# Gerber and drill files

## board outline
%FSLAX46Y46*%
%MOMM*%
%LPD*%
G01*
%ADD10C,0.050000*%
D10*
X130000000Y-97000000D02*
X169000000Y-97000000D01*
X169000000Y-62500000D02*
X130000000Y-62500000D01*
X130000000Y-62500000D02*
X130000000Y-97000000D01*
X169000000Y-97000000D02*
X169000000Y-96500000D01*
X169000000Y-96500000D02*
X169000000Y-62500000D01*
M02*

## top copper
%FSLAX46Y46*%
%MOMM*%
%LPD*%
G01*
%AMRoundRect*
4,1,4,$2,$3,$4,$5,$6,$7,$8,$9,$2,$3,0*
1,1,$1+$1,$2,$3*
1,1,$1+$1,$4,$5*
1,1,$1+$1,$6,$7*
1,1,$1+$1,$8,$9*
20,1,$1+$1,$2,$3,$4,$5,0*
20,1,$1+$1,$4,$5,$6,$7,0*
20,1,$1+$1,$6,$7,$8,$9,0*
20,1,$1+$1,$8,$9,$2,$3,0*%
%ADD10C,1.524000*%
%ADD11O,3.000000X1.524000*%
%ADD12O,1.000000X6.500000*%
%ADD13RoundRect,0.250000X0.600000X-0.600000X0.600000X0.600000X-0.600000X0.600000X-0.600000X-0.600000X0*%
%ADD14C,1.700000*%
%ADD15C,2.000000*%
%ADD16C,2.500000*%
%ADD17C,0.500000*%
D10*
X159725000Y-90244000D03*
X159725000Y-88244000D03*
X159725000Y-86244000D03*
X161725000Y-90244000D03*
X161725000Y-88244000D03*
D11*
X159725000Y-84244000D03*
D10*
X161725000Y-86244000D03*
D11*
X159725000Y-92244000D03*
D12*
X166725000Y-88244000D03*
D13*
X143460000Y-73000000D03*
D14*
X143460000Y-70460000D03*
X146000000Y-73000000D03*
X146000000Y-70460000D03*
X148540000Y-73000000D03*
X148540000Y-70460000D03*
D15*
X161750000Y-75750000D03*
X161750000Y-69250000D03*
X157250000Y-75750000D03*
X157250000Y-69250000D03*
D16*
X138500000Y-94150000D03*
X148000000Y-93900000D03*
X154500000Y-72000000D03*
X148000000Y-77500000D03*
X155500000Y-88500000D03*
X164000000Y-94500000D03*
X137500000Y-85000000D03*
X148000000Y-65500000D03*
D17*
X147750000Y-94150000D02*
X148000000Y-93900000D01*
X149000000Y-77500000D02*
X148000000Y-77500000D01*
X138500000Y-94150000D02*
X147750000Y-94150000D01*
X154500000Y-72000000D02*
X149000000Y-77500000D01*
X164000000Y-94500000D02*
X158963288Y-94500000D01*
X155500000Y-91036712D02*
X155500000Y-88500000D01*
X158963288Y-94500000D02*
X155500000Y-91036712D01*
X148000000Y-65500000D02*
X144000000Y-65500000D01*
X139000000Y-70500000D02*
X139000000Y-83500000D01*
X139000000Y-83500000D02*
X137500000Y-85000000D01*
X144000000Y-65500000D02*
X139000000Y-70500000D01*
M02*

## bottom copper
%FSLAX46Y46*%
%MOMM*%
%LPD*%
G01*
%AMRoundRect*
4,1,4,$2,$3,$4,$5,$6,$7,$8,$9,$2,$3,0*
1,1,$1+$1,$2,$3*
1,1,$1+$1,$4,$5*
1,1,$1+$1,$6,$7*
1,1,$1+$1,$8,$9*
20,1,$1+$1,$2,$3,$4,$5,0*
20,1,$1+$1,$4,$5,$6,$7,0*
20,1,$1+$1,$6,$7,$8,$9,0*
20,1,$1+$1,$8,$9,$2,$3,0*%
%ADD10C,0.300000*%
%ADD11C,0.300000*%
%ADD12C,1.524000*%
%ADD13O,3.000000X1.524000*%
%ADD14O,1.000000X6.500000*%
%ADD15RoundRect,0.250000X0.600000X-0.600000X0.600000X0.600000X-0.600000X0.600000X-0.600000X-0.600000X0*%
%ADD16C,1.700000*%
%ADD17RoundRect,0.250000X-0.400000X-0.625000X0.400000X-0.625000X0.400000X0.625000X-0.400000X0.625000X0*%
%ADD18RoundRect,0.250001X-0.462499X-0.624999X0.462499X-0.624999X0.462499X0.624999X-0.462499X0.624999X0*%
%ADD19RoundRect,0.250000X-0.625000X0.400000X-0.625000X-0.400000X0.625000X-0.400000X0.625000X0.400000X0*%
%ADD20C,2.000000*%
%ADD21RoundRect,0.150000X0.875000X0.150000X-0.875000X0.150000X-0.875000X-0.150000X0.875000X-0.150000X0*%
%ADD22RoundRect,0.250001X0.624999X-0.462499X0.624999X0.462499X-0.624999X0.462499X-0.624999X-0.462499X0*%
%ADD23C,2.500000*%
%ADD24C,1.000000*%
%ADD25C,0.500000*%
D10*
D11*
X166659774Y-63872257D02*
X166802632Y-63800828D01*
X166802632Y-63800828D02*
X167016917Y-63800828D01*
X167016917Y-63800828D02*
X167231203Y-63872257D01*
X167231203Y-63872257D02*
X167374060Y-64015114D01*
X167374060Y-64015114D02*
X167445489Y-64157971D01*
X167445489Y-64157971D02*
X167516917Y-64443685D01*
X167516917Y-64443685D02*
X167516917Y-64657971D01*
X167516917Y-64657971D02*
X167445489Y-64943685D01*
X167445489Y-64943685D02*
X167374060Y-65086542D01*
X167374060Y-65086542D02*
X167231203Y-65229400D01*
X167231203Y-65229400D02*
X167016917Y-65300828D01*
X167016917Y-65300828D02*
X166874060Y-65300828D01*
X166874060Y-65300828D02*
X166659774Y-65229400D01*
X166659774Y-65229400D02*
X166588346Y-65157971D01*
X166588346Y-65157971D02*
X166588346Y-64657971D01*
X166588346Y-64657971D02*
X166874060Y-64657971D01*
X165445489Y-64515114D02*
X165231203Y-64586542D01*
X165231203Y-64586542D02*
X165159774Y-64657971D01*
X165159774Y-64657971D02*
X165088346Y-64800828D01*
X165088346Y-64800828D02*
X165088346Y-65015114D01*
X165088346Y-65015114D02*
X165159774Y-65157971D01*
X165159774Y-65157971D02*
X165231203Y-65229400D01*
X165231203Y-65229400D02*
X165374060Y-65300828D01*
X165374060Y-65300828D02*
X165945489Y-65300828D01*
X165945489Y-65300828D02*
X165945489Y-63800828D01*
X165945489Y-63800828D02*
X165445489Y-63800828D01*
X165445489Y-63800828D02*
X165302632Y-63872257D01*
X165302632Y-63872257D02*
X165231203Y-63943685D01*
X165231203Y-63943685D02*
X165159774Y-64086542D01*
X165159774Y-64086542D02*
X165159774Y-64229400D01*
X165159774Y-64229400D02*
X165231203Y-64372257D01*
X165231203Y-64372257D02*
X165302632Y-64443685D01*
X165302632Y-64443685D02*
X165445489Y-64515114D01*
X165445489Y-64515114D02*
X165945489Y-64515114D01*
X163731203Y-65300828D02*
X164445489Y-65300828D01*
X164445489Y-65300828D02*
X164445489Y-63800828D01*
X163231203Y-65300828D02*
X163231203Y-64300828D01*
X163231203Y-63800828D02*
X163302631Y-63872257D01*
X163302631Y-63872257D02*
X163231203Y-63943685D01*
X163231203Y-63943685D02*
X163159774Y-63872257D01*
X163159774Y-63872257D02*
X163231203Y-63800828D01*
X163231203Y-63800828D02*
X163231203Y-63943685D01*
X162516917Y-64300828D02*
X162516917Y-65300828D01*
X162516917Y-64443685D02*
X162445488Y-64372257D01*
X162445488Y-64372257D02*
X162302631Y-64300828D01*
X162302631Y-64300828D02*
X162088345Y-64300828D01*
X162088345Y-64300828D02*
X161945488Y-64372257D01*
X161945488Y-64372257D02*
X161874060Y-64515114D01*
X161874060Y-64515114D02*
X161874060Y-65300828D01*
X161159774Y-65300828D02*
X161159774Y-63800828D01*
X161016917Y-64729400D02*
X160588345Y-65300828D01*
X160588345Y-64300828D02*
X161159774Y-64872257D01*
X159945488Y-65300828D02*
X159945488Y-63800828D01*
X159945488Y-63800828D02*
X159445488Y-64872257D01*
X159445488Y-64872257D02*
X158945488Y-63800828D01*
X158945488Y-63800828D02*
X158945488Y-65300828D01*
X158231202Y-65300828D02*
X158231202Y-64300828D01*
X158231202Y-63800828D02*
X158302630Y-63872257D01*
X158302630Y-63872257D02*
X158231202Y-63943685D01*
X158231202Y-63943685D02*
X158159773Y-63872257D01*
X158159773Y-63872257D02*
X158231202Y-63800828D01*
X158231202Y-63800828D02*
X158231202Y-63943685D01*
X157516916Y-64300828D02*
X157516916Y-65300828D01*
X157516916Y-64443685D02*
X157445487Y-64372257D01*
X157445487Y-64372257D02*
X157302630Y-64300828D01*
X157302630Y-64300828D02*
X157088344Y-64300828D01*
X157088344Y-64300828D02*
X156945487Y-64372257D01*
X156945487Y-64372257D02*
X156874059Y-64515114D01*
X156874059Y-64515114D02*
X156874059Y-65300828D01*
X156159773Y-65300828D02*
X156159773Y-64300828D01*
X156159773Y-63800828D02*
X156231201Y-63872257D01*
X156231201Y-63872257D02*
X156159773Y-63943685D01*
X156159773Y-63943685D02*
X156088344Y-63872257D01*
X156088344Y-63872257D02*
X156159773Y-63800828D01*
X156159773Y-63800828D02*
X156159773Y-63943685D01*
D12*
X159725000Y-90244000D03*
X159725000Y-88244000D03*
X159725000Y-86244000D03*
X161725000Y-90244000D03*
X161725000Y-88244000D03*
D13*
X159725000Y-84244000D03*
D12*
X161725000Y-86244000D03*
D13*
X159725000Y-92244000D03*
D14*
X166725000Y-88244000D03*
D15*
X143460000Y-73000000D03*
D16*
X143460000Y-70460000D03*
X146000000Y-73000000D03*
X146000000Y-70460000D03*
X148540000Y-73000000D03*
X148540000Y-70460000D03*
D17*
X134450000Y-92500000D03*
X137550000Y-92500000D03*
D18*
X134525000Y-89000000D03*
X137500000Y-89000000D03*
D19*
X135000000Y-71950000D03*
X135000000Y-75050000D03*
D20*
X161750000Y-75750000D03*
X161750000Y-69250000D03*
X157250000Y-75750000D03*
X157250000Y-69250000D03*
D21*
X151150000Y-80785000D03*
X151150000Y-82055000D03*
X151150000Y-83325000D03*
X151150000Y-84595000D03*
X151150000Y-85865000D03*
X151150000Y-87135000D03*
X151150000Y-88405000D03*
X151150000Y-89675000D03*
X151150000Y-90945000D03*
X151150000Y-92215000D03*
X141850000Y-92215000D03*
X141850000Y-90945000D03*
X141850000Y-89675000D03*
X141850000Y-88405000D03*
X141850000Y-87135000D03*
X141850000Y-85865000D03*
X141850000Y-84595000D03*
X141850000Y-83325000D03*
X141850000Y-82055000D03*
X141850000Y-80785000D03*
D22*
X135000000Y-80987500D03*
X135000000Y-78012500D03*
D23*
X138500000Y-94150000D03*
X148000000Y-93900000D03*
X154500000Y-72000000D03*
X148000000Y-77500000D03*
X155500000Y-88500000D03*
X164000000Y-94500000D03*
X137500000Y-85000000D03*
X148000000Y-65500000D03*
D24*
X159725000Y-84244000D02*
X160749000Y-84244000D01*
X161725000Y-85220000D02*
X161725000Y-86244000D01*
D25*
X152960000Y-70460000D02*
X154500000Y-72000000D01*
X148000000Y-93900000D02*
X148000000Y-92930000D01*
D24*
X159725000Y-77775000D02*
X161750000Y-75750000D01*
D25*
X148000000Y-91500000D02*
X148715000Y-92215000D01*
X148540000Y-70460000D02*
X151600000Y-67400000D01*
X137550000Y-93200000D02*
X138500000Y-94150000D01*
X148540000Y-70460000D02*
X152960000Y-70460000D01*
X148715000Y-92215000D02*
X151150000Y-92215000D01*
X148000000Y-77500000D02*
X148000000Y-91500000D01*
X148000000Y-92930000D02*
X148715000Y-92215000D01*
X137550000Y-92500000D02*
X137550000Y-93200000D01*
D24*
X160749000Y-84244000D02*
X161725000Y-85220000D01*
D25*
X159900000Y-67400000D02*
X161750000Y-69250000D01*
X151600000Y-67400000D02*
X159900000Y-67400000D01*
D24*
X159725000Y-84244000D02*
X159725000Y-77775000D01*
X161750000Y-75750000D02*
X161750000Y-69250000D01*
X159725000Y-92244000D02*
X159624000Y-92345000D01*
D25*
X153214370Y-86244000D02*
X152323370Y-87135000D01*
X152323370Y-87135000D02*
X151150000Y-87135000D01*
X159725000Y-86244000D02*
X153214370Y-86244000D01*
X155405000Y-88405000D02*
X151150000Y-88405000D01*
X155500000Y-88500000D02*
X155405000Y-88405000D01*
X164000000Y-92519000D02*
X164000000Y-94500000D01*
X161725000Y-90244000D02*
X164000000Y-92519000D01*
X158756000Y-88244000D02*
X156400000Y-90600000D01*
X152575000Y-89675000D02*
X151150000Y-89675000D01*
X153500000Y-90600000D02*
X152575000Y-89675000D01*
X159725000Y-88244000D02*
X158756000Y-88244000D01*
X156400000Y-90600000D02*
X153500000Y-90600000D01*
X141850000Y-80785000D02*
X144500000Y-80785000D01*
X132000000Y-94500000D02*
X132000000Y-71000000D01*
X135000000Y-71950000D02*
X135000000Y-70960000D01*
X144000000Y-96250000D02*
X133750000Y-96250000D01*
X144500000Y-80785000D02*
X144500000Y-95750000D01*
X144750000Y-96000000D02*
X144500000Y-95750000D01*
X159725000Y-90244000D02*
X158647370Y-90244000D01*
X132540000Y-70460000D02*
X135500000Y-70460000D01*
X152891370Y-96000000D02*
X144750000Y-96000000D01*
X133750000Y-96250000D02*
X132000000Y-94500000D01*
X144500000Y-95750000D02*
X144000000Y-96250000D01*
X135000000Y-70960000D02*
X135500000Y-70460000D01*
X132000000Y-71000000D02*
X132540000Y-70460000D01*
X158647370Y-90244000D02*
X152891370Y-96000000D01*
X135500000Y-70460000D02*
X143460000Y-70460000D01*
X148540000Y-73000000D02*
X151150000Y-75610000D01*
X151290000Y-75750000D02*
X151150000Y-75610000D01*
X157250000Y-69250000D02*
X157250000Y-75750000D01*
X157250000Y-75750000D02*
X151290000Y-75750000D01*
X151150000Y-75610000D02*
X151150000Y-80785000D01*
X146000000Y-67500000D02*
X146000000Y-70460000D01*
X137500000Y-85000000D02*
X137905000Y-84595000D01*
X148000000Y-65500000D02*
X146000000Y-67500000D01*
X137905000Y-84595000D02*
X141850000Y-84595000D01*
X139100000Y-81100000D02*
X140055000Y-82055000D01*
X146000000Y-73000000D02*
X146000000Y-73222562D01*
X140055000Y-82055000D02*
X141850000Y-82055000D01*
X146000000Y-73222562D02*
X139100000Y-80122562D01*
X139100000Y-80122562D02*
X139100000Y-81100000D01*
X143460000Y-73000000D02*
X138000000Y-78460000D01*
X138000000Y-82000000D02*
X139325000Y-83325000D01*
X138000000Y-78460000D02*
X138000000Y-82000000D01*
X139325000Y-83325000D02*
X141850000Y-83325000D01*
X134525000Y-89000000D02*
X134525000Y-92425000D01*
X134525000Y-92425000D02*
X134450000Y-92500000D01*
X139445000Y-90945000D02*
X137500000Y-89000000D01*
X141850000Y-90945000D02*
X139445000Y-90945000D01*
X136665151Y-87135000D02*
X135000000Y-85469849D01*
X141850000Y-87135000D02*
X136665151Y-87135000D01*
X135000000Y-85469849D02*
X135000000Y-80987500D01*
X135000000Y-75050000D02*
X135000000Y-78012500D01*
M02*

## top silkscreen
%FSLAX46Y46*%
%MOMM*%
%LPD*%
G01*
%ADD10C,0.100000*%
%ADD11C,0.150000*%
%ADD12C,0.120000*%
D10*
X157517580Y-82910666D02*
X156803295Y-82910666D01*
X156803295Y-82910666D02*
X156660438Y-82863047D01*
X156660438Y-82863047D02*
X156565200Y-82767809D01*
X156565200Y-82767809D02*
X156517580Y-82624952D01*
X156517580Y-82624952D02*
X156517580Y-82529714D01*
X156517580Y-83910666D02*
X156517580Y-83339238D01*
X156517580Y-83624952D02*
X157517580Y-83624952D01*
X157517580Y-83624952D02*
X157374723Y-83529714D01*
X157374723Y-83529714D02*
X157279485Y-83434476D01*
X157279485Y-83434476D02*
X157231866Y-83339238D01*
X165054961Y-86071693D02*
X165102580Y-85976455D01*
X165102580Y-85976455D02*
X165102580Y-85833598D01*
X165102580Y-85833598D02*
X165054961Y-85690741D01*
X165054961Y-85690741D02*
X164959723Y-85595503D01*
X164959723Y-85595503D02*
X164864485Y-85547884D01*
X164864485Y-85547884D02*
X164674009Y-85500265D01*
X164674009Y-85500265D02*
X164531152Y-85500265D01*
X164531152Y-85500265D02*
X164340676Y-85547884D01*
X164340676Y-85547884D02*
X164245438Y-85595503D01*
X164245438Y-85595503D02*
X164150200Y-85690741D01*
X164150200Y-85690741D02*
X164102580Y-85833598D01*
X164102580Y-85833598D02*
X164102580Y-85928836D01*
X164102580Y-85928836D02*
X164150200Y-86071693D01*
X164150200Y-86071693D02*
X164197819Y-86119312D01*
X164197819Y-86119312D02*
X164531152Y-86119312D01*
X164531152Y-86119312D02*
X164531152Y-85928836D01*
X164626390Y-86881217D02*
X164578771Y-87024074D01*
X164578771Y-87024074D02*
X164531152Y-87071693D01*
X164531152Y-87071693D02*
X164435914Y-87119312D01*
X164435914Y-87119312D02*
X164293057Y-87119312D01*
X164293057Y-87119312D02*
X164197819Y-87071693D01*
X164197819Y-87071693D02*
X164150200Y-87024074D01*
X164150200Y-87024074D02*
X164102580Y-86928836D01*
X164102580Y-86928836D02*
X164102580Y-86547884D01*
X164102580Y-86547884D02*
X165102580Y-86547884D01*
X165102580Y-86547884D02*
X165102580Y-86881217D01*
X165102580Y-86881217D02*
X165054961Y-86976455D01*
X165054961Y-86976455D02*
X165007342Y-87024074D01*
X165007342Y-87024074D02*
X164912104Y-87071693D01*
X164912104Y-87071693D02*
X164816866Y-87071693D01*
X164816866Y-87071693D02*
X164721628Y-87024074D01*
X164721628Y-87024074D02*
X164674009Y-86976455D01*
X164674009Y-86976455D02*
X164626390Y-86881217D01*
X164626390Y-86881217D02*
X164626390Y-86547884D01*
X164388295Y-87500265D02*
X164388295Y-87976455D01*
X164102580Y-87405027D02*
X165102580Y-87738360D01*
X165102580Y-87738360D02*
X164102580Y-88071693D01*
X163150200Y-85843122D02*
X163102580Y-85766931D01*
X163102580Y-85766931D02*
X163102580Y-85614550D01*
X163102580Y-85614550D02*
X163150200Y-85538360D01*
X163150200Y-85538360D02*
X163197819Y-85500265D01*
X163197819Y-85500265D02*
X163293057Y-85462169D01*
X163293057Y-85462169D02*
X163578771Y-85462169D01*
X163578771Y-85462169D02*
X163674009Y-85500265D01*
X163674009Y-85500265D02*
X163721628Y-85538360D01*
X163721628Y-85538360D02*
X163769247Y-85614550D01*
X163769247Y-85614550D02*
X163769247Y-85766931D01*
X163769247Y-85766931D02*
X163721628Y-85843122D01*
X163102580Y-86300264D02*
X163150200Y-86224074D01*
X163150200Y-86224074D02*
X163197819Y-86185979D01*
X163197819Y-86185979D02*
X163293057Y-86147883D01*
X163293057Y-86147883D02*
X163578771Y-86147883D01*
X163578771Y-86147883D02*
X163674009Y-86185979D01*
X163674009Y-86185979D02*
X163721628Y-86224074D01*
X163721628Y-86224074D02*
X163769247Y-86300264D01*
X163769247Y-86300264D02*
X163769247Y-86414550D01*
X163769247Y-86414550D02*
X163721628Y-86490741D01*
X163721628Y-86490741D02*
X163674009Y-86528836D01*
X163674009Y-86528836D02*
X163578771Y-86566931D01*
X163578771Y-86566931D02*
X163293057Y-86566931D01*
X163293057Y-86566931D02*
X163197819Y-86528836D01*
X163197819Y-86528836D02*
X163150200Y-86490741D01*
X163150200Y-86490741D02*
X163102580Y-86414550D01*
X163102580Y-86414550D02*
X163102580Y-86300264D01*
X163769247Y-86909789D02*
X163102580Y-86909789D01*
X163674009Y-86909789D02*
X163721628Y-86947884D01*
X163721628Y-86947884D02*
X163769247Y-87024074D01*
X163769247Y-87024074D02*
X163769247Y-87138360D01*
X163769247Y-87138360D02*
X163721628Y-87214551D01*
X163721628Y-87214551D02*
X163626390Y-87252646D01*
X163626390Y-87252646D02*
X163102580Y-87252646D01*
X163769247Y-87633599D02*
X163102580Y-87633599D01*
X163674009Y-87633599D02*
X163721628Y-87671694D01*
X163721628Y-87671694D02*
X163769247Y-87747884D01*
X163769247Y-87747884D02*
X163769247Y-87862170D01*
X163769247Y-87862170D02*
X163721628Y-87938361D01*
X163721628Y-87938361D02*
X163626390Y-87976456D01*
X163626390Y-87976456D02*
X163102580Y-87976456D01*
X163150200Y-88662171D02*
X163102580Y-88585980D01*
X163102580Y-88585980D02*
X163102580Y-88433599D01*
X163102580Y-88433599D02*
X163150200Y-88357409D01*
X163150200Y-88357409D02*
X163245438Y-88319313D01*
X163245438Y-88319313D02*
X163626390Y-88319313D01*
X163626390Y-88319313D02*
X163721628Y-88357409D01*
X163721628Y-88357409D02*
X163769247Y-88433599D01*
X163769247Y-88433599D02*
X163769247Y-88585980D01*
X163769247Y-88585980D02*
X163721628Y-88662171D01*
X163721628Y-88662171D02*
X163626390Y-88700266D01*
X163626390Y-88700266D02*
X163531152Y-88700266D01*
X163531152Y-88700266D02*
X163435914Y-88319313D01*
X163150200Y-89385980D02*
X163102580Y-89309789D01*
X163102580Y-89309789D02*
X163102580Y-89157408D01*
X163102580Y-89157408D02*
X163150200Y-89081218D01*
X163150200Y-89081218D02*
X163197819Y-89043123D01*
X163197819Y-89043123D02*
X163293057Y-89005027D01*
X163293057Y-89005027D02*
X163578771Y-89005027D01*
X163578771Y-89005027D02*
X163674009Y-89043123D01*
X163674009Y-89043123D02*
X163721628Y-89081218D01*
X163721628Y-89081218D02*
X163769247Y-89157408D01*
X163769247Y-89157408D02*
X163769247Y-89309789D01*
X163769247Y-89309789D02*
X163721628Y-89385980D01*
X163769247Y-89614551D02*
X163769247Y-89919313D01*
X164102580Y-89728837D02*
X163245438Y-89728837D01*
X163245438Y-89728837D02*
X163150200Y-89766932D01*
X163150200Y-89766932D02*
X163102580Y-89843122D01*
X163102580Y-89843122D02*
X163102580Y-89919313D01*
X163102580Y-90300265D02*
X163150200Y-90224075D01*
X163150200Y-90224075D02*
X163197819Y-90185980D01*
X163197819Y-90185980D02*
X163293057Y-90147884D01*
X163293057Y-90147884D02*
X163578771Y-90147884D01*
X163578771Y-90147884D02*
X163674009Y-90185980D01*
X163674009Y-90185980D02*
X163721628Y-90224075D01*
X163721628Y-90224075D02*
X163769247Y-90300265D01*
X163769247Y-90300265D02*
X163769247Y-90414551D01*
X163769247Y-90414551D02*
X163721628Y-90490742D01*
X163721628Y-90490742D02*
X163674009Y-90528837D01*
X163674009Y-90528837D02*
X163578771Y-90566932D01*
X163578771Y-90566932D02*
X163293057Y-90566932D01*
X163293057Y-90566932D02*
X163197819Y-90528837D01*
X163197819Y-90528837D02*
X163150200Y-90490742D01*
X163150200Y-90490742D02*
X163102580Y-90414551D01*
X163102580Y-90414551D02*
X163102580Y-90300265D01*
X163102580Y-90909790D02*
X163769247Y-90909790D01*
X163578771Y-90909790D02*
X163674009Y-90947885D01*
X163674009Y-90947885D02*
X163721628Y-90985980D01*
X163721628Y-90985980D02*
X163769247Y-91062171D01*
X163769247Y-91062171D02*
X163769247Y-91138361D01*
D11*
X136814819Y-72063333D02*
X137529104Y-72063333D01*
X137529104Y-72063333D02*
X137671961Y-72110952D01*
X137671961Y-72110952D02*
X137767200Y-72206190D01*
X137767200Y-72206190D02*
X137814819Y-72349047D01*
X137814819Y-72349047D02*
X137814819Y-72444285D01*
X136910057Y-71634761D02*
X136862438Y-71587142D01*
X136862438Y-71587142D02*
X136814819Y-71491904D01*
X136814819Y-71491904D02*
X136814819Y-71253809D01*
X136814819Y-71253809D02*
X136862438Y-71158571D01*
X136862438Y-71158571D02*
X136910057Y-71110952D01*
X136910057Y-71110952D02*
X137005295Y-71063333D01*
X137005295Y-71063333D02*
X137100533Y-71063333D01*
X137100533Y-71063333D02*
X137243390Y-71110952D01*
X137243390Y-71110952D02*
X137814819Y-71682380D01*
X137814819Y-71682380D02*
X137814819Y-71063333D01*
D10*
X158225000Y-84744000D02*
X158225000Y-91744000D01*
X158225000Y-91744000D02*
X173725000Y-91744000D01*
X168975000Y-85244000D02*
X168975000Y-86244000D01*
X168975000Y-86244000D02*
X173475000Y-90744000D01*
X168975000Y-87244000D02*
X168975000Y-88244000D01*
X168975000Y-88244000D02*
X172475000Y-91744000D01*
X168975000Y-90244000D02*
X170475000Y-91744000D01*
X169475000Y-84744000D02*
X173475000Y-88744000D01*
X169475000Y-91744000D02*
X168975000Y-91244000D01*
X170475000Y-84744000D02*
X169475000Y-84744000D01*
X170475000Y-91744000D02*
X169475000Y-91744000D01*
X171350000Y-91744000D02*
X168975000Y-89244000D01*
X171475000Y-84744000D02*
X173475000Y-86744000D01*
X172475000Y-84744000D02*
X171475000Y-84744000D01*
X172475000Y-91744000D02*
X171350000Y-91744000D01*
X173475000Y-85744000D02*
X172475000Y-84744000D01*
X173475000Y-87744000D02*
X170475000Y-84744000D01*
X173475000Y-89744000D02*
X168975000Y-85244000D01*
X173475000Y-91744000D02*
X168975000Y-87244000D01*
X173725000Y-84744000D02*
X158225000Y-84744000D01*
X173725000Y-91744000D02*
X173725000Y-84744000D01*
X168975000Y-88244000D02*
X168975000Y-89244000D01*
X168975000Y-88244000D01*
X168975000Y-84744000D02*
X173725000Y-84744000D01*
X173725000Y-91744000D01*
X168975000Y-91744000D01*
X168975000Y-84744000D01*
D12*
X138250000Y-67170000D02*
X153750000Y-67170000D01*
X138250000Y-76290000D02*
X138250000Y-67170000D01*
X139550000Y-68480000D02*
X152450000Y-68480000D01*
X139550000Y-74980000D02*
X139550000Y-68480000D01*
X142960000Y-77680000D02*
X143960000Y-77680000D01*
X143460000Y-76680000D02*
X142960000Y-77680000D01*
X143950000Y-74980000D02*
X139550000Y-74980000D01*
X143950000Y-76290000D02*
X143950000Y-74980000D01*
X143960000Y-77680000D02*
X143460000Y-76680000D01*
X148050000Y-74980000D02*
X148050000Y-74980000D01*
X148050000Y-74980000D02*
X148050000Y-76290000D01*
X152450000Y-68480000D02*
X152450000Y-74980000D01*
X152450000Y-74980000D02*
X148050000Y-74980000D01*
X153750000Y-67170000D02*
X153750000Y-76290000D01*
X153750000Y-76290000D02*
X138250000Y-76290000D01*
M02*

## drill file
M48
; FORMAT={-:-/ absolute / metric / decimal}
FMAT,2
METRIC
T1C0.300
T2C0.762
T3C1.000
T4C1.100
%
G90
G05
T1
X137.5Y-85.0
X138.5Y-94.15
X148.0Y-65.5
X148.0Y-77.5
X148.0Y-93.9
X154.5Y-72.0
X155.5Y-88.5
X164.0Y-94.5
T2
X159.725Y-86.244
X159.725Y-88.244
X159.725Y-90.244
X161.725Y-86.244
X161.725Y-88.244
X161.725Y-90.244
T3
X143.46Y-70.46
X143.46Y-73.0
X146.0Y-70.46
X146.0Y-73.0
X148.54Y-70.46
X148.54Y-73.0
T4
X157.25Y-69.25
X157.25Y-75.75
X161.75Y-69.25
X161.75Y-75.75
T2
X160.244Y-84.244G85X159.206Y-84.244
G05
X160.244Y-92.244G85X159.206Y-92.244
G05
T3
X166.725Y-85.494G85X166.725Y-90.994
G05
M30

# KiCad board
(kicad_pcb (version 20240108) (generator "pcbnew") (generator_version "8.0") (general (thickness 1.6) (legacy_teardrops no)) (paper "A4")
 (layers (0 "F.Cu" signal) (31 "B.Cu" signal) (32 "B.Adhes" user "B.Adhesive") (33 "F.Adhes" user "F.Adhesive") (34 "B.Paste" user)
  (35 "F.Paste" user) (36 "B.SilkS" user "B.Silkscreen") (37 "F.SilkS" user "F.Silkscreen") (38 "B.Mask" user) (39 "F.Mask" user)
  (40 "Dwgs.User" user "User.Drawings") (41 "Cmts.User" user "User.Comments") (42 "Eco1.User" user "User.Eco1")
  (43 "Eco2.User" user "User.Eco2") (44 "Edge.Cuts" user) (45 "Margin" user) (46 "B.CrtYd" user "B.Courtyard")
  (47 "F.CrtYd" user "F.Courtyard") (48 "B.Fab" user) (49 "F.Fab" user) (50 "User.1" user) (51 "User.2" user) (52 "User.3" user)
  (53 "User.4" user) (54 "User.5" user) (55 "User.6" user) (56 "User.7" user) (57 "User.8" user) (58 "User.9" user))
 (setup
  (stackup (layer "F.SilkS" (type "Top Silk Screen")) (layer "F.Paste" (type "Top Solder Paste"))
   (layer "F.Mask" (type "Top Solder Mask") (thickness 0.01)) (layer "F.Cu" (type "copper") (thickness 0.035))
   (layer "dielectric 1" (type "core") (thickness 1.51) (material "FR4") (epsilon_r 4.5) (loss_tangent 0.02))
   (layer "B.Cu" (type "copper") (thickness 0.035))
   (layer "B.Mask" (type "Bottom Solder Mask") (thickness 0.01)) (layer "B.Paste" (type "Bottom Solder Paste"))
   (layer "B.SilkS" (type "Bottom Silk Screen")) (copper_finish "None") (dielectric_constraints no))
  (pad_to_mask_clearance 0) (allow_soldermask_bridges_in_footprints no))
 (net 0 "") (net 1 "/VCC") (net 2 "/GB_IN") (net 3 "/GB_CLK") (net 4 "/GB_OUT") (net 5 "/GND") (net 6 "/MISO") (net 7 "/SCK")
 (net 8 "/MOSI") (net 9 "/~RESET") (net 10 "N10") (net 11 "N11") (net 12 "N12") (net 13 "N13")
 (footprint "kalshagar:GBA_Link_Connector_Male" (layer "F.Cu") (at 156.475 83.244 -90)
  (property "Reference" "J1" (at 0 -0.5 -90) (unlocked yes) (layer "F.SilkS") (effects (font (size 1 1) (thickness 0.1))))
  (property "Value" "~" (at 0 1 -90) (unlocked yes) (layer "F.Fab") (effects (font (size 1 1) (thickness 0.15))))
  (fp_line (start 1.5 -1.75) (end 8.5 -1.75) (stroke (width 0.1) (type default)) (layer "F.SilkS"))
  (fp_line (start 8.5 -1.75) (end 8.5 -17.25) (stroke (width 0.1) (type default)) (layer "F.SilkS"))
  (fp_line (start 2 -12.5) (end 3 -12.5) (stroke (width 0.1) (type default)) (layer "F.SilkS"))
  (fp_line (start 3 -12.5) (end 7.5 -17) (stroke (width 0.1) (type default)) (layer "F.SilkS"))
  (fp_line (start 4 -12.5) (end 5 -12.5) (stroke (width 0.1) (type default)) (layer "F.SilkS"))
  (fp_line (start 5 -12.5) (end 8.5 -16) (stroke (width 0.1) (type default)) (layer "F.SilkS"))
  (fp_line (start 7 -12.5) (end 8.5 -14) (stroke (width 0.1) (type default)) (layer "F.SilkS"))
  (fp_line (start 1.5 -13) (end 5.5 -17) (stroke (width 0.1) (type default)) (layer "F.SilkS"))
  (fp_line (start 8.5 -13) (end 8 -12.5) (stroke (width 0.1) (type default)) (layer "F.SilkS"))
  (fp_line (start 1.5 -14) (end 1.5 -13) (stroke (width 0.1) (type default)) (layer "F.SilkS"))
  (fp_line (start 8.5 -14) (end 8.5 -13) (stroke (width 0.1) (type default)) (layer "F.SilkS"))
  (fp_line (start 8.5 -14.875) (end 6 -12.5) (stroke (width 0.1) (type default)) (layer "F.SilkS"))
  (fp_line (start 1.5 -15) (end 3.5 -17) (stroke (width 0.1) (type default)) (layer "F.SilkS"))
  (fp_line (start 1.5 -16) (end 1.5 -15) (stroke (width 0.1) (type default)) (layer "F.SilkS"))
  (fp_line (start 8.5 -16) (end 8.5 -14.875) (stroke (width 0.1) (type default)) (layer "F.SilkS"))
  (fp_line (start 2.5 -17) (end 1.5 -16) (stroke (width 0.1) (type default)) (layer "F.SilkS"))
  (fp_line (start 4.5 -17) (end 1.5 -14) (stroke (width 0.1) (type default)) (layer "F.SilkS"))
  (fp_line (start 6.5 -17) (end 2 -12.5) (stroke (width 0.1) (type default)) (layer "F.SilkS"))
  (fp_line (start 8.5 -17) (end 4 -12.5) (stroke (width 0.1) (type default)) (layer "F.SilkS"))
  (fp_line (start 1.5 -17.25) (end 1.5 -1.75) (stroke (width 0.1) (type default)) (layer "F.SilkS"))
  (fp_line (start 8.5 -17.25) (end 1.5 -17.25) (stroke (width 0.1) (type default)) (layer "F.SilkS"))
  (fp_rect (start 5 -12.5) (end 6 -12.5) (stroke (width 0.1) (type default)) (fill none) (layer "F.SilkS"))
  (fp_rect (start 1.5 -17.25) (end 8.5 -12.5) (stroke (width 0.1) (type solid)) (fill none) (layer "F.SilkS"))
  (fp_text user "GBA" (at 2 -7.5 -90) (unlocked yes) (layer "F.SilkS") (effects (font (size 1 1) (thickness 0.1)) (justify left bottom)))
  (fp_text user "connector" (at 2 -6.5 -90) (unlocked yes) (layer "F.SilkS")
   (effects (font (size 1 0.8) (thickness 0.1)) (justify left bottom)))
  (pad "1" thru_hole circle (at 7 -3.25 270) (size 1.524 1.524) (drill 0.762) (layers "*.Cu" "*.Mask") (remove_unused_layers no)
   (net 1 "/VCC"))
  (pad "2" thru_hole circle (at 5 -3.25 270) (size 1.524 1.524) (drill 0.762) (layers "*.Cu" "*.Mask") (remove_unused_layers no)
   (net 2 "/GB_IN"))
  (pad "3" thru_hole circle (at 3 -3.25 270) (size 1.524 1.524) (drill 0.762) (layers "*.Cu" "*.Mask") (remove_unused_layers no)
   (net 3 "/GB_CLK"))
  (pad "4" thru_hole circle (at 7 -5.25 270) (size 1.524 1.524) (drill 0.762) (layers "*.Cu" "*.Mask") (remove_unused_layers no)
   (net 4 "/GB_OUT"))
  (pad "5" thru_hole circle (at 5 -5.25 270) (size 1.524 1.524) (drill 0.762) (layers "*.Cu" "*.Mask") (remove_unused_layers no))
  (pad "6" thru_hole oval (at 1 -3.25 270) (size 1.524 3) (drill oval 0.762 1.8) (layers "*.Cu" "*.Mask") (remove_unused_layers no)
   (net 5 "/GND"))
  (pad "6" thru_hole circle (at 3 -5.25 270) (size 1.524 1.524) (drill 0.762) (layers "*.Cu" "*.Mask") (remove_unused_layers no)
   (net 5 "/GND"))
  (pad "6" thru_hole oval (at 9 -3.25 270) (size 1.524 3) (drill oval 0.762 1.8) (layers "*.Cu" "*.Mask") (remove_unused_layers no)
   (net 5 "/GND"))
  (pad "7" thru_hole oval (at 5 -10.25) (size 1 6.5) (drill oval 1 6.5) (layers "*.Cu" "*.Mask") (remove_unused_layers no)))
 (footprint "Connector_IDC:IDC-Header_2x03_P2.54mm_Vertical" (layer "F.Cu") (at 143.46 73 90)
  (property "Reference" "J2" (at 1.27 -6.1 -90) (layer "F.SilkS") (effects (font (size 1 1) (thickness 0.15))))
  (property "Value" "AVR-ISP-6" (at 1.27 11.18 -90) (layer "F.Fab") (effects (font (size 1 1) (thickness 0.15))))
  (fp_line (start 5.83 -5.21) (end 5.83 10.29) (stroke (width 0.12) (type solid)) (layer "F.SilkS"))
  (fp_line (start -3.29 -5.21) (end 5.83 -5.21) (stroke (width 0.12) (type solid)) (layer "F.SilkS"))
  (fp_line (start 4.52 -3.91) (end 4.52 8.99) (stroke (width 0.12) (type solid)) (layer "F.SilkS"))
  (fp_line (start -1.98 -3.91) (end 4.52 -3.91) (stroke (width 0.12) (type solid)) (layer "F.SilkS"))
  (fp_line (start -4.68 -0.5) (end -4.68 0.5) (stroke (width 0.12) (type solid)) (layer "F.SilkS"))
  (fp_line (start -3.68 0) (end -4.68 -0.5) (stroke (width 0.12) (type solid)) (layer "F.SilkS"))
  (fp_line (start -1.98 0.49) (end -1.98 -3.91) (stroke (width 0.12) (type solid)) (layer "F.SilkS"))
  (fp_line (start -3.29 0.49) (end -1.98 0.49) (stroke (width 0.12) (type solid)) (layer "F.SilkS"))
  (fp_line (start -4.68 0.5) (end -3.68 0) (stroke (width 0.12) (type solid)) (layer "F.SilkS"))
  (fp_line (start -1.98 4.59) (end -1.98 4.59) (stroke (width 0.12) (type solid)) (layer "F.SilkS"))
  (fp_line (start -1.98 4.59) (end -3.29 4.59) (stroke (width 0.12) (type solid)) (layer "F.SilkS"))
  (fp_line (start 4.52 8.99) (end -1.98 8.99) (stroke (width 0.12) (type solid)) (layer "F.SilkS"))
  (fp_line (start -1.98 8.99) (end -1.98 4.59) (stroke (width 0.12) (type solid)) (layer "F.SilkS"))
  (fp_line (start 5.83 10.29) (end -3.29 10.29) (stroke (width 0.12) (type solid)) (layer "F.SilkS"))
  (fp_line (start -3.29 10.29) (end -3.29 -5.21) (stroke (width 0.12) (type solid)) (layer "F.SilkS"))
  (pad "1" thru_hole roundrect (at 0 0 90) (size 1.7 1.7) (drill 1) (layers "*.Cu" "*.Mask") (remove_unused_layers no)
   (roundrect_rratio 0.147059) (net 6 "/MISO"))
  (pad "2" thru_hole circle (at 2.54 0 90) (size 1.7 1.7) (drill 1) (layers "*.Cu" "*.Mask") (remove_unused_layers no) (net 1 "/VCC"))
  (pad "3" thru_hole circle (at 0 2.54 90) (size 1.7 1.7) (drill 1) (layers "*.Cu" "*.Mask") (remove_unused_layers no) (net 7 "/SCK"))
  (pad "4" thru_hole circle (at 2.54 2.54 90) (size 1.7 1.7) (drill 1) (layers "*.Cu" "*.Mask") (remove_unused_layers no) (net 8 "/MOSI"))
  (pad "5" thru_hole circle (at 0 5.08 90) (size 1.7 1.7) (drill 1) (layers "*.Cu" "*.Mask") (remove_unused_layers no) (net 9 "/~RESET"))
  (pad "6" thru_hole circle (at 2.54 5.08 90) (size 1.7 1.7) (drill 1) (layers "*.Cu" "*.Mask") (remove_unused_layers no) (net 5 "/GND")))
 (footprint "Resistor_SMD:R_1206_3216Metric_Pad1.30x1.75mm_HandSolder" (layer "B.Cu") (at 136 92.5)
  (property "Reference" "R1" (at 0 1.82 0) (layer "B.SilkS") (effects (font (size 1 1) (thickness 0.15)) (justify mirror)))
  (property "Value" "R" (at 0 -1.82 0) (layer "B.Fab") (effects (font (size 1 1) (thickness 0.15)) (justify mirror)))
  (pad "1" smd roundrect (at -1.55 0) (size 1.3 1.75) (layers "B.Cu" "B.Paste" "B.Mask") (roundrect_rratio 0.192308) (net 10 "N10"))
  (pad "2" smd roundrect (at 1.55 0) (size 1.3 1.75) (layers "B.Cu" "B.Paste" "B.Mask") (roundrect_rratio 0.192308) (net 5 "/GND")))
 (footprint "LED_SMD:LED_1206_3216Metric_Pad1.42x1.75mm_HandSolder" (layer "B.Cu") (at 136.0125 89)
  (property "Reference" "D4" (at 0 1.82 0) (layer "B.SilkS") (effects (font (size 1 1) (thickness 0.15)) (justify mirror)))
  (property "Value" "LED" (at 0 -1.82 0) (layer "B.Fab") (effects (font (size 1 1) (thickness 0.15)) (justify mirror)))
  (pad "1" smd roundrect (at -1.4875 0) (size 1.425 1.75) (layers "B.Cu" "B.Paste" "B.Mask") (roundrect_rratio 0.175439) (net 10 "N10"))
  (pad "2" smd roundrect (at 1.4875 0) (size 1.425 1.75) (layers "B.Cu" "B.Paste" "B.Mask") (roundrect_rratio 0.175439) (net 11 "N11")))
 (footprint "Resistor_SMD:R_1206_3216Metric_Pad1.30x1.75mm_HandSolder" (layer "B.Cu") (at 135 73.5 -90)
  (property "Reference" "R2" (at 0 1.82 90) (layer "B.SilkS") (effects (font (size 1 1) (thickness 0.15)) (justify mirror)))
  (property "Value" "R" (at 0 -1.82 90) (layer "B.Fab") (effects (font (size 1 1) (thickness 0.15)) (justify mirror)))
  (pad "1" smd roundrect (at -1.55 0 270) (size 1.3 1.75) (layers "B.Cu" "B.Paste" "B.Mask") (roundrect_rratio 0.192308) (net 1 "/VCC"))
  (pad "2" smd roundrect (at 1.55 0 270) (size 1.3 1.75) (layers "B.Cu" "B.Paste" "B.Mask") (roundrect_rratio 0.192308) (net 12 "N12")))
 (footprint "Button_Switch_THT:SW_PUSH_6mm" (layer "B.Cu") (at 161.75 75.75 90)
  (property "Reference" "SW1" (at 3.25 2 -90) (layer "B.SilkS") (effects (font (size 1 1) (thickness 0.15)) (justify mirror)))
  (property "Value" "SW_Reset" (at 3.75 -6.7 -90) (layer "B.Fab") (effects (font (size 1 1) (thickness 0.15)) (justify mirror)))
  (pad "1" thru_hole circle (at 0 0) (size 2 2) (drill 1.1) (layers "*.Cu" "*.Mask") (remove_unused_layers no) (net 5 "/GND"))
  (pad "1" thru_hole circle (at 6.5 0) (size 2 2) (drill 1.1) (layers "*.Cu" "*.Mask") (remove_unused_layers no) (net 5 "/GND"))
  (pad "2" thru_hole circle (at 0 -4.5) (size 2 2) (drill 1.1) (layers "*.Cu" "*.Mask") (remove_unused_layers no) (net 9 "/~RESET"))
  (pad "2" thru_hole circle (at 6.5 -4.5) (size 2 2) (drill 1.1) (layers "*.Cu" "*.Mask") (remove_unused_layers no) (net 9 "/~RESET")))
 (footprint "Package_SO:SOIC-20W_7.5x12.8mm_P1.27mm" (layer "B.Cu") (at 146.5 86.5 180)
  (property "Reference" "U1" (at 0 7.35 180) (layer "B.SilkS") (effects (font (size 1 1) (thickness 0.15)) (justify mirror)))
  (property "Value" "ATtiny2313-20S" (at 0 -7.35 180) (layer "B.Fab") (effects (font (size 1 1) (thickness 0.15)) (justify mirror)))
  (pad "1" smd roundrect (at -4.65 5.715 180) (size 2.05 0.6) (layers "B.Cu" "B.Paste" "B.Mask") (roundrect_rratio 0.25) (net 9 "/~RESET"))
  (pad "2" smd roundrect (at -4.65 4.445 180) (size 2.05 0.6) (layers "B.Cu" "B.Paste" "B.Mask") (roundrect_rratio 0.25))
  (pad "3" smd roundrect (at -4.65 3.175 180) (size 2.05 0.6) (layers "B.Cu" "B.Paste" "B.Mask") (roundrect_rratio 0.25))
  (pad "4" smd roundrect (at -4.65 1.905 180) (size 2.05 0.6) (layers "B.Cu" "B.Paste" "B.Mask") (roundrect_rratio 0.25))
  (pad "5" smd roundrect (at -4.65 0.635 180) (size 2.05 0.6) (layers "B.Cu" "B.Paste" "B.Mask") (roundrect_rratio 0.25))
  (pad "6" smd roundrect (at -4.65 -0.635 180) (size 2.05 0.6) (layers "B.Cu" "B.Paste" "B.Mask") (roundrect_rratio 0.25) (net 3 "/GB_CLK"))
  (pad "7" smd roundrect (at -4.65 -1.905 180) (size 2.05 0.6) (layers "B.Cu" "B.Paste" "B.Mask") (roundrect_rratio 0.25) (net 4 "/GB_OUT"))
  (pad "8" smd roundrect (at -4.65 -3.175 180) (size 2.05 0.6) (layers "B.Cu" "B.Paste" "B.Mask") (roundrect_rratio 0.25) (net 2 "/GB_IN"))
  (pad "9" smd roundrect (at -4.65 -4.445 180) (size 2.05 0.6) (layers "B.Cu" "B.Paste" "B.Mask") (roundrect_rratio 0.25))
  (pad "10" smd roundrect (at -4.65 -5.715 180) (size 2.05 0.6) (layers "B.Cu" "B.Paste" "B.Mask") (roundrect_rratio 0.25) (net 5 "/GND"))
  (pad "11" smd roundrect (at 4.65 -5.715 180) (size 2.05 0.6) (layers "B.Cu" "B.Paste" "B.Mask") (roundrect_rratio 0.25))
  (pad "12" smd roundrect (at 4.65 -4.445 180) (size 2.05 0.6) (layers "B.Cu" "B.Paste" "B.Mask") (roundrect_rratio 0.25) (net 11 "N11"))
  (pad "13" smd roundrect (at 4.65 -3.175 180) (size 2.05 0.6) (layers "B.Cu" "B.Paste" "B.Mask") (roundrect_rratio 0.25))
  (pad "14" smd roundrect (at 4.65 -1.905 180) (size 2.05 0.6) (layers "B.Cu" "B.Paste" "B.Mask") (roundrect_rratio 0.25))
  (pad "15" smd roundrect (at 4.65 -0.635 180) (size 2.05 0.6) (layers "B.Cu" "B.Paste" "B.Mask") (roundrect_rratio 0.25) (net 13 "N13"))
  (pad "16" smd roundrect (at 4.65 0.635 180) (size 2.05 0.6) (layers "B.Cu" "B.Paste" "B.Mask") (roundrect_rratio 0.25))
  (pad "17" smd roundrect (at 4.65 1.905 180) (size 2.05 0.6) (layers "B.Cu" "B.Paste" "B.Mask") (roundrect_rratio 0.25) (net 8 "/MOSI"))
  (pad "18" smd roundrect (at 4.65 3.175 180) (size 2.05 0.6) (layers "B.Cu" "B.Paste" "B.Mask") (roundrect_rratio 0.25) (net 6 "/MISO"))
  (pad "19" smd roundrect (at 4.65 4.445 180) (size 2.05 0.6) (layers "B.Cu" "B.Paste" "B.Mask") (roundrect_rratio 0.25) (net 7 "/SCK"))
  (pad "20" smd roundrect (at 4.65 5.715 180) (size 2.05 0.6) (layers "B.Cu" "B.Paste" "B.Mask") (roundrect_rratio 0.25) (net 1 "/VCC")))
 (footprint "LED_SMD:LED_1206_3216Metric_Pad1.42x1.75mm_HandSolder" (layer "B.Cu") (at 135 79.5 90)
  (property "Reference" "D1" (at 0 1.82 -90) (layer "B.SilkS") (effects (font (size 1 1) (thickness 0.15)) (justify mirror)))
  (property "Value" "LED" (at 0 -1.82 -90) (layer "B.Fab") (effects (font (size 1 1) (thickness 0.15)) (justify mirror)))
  (pad "1" smd roundrect (at -1.4875 0 90) (size 1.425 1.75) (layers "B.Cu" "B.Paste" "B.Mask") (roundrect_rratio 0.175439) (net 13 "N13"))
  (pad "2" smd roundrect (at 1.4875 0 90) (size 1.425 1.75) (layers "B.Cu" "B.Paste" "B.Mask") (roundrect_rratio 0.175439) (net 12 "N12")))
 (gr_line (start 130 97) (end 169 97) (stroke (width 0.05) (type default)) (layer "Edge.Cuts"))
 (gr_line (start 169 62.5) (end 130 62.5) (stroke (width 0.05) (type default)) (layer "Edge.Cuts"))
 (gr_line (start 130 62.5) (end 130 97) (stroke (width 0.05) (type default)) (layer "Edge.Cuts"))
 (gr_line (start 169 97) (end 169 96.5) (stroke (width 0.05) (type default)) (layer "Edge.Cuts"))
 (gr_line (start 169 96.5) (end 169 62.5) (stroke (width 0.05) (type default)) (layer "Edge.Cuts"))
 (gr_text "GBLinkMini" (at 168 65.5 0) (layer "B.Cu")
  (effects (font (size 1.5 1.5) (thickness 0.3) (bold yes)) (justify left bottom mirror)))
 (segment (start 147.75 94.15) (end 148 93.9) (width 0.5) (layer "F.Cu") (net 5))
 (segment (start 149 77.5) (end 148 77.5) (width 0.5) (layer "F.Cu") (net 5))
 (segment (start 138.5 94.15) (end 147.75 94.15) (width 0.5) (layer "F.Cu") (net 5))
 (segment (start 154.5 72) (end 149 77.5) (width 0.5) (layer "F.Cu") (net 5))
 (via (at 138.5 94.15) (size 2.5) (drill 0.3) (layers "F.Cu" "B.Cu") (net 5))
 (via (at 148 93.9) (size 2.5) (drill 0.3) (layers "F.Cu" "B.Cu") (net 5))
 (via (at 154.5 72) (size 2.5) (drill 0.3) (layers "F.Cu" "B.Cu") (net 5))
 (via (at 148 77.5) (size 2.5) (drill 0.3) (layers "F.Cu" "B.Cu") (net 5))
 (segment (start 159.725 84.244) (end 160.749 84.244) (width 1) (layer "B.Cu") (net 5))
 (segment (start 161.725 85.22) (end 161.725 86.244) (width 1) (layer "B.Cu") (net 5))
 (segment (start 152.96 70.46) (end 154.5 72) (width 0.5) (layer "B.Cu") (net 5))
 (segment (start 148 93.9) (end 148 92.93) (width 0.5) (layer "B.Cu") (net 5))
 (segment (start 159.725 77.775) (end 161.75 75.75) (width 1) (layer "B.Cu") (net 5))
 (segment (start 148 91.5) (end 148.715 92.215) (width 0.5) (layer "B.Cu") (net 5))
 (segment (start 148.54 70.46) (end 151.6 67.4) (width 0.5) (layer "B.Cu") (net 5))
 (segment (start 137.55 93.2) (end 138.5 94.15) (width 0.5) (layer "B.Cu") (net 5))
 (segment (start 148.54 70.46) (end 152.96 70.46) (width 0.5) (layer "B.Cu") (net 5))
 (segment (start 148.715 92.215) (end 151.15 92.215) (width 0.5) (layer "B.Cu") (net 5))
 (segment (start 148 77.5) (end 148 91.5) (width 0.5) (layer "B.Cu") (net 5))
 (segment (start 148 92.93) (end 148.715 92.215) (width 0.5) (layer "B.Cu") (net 5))
 (segment (start 137.55 92.5) (end 137.55 93.2) (width 0.5) (layer "B.Cu") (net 5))
 (segment (start 160.749 84.244) (end 161.725 85.22) (width 1) (layer "B.Cu") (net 5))
 (segment (start 159.9 67.4) (end 161.75 69.25) (width 0.5) (layer "B.Cu") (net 5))
 (segment (start 151.6 67.4) (end 159.9 67.4) (width 0.5) (layer "B.Cu") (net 5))
 (segment (start 159.725 84.244) (end 159.725 77.775) (width 1) (layer "B.Cu") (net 5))
 (segment (start 161.75 75.75) (end 161.75 69.25) (width 1) (layer "B.Cu") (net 5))
 (segment (start 159.725 92.244) (end 159.624 92.345) (width 1) (layer "B.Cu") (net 5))
 (segment (start 153.21437 86.244) (end 152.32337 87.135) (width 0.5) (layer "B.Cu") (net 3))
 (segment (start 152.32337 87.135) (end 151.15 87.135) (width 0.5) (layer "B.Cu") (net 3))
 (segment (start 159.725 86.244) (end 153.21437 86.244) (width 0.5) (layer "B.Cu") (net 3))
 (segment (start 164 94.5) (end 158.963288 94.5) (width 0.5) (layer "F.Cu") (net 4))
 (segment (start 155.5 91.036712) (end 155.5 88.5) (width 0.5) (layer "F.Cu") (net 4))
 (segment (start 158.963288 94.5) (end 155.5 91.036712) (width 0.5) (layer "F.Cu") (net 4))
 (via (at 155.5 88.5) (size 2.5) (drill 0.3) (layers "F.Cu" "B.Cu") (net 4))
 (via (at 164 94.5) (size 2.5) (drill 0.3) (layers "F.Cu" "B.Cu") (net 4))
 (segment (start 155.405 88.405) (end 151.15 88.405) (width 0.5) (layer "B.Cu") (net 4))
 (segment (start 155.5 88.5) (end 155.405 88.405) (width 0.5) (layer "B.Cu") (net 4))
 (segment (start 164 92.519) (end 164 94.5) (width 0.5) (layer "B.Cu") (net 4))
 (segment (start 161.725 90.244) (end 164 92.519) (width 0.5) (layer "B.Cu") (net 4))
 (segment (start 158.756 88.244) (end 156.4 90.6) (width 0.5) (layer "B.Cu") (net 2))
 (segment (start 152.575 89.675) (end 151.15 89.675) (width 0.5) (layer "B.Cu") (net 2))
 (segment (start 153.5 90.6) (end 152.575 89.675) (width 0.5) (layer "B.Cu") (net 2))
 (segment (start 159.725 88.244) (end 158.756 88.244) (width 0.5) (layer "B.Cu") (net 2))
 (segment (start 156.4 90.6) (end 153.5 90.6) (width 0.5) (layer "B.Cu") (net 2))
 (segment (start 141.85 80.785) (end 144.5 80.785) (width 0.5) (layer "B.Cu") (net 1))
 (segment (start 132 94.5) (end 132 71) (width 0.5) (layer "B.Cu") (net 1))
 (segment (start 135 71.95) (end 135 70.96) (width 0.5) (layer "B.Cu") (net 1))
 (segment (start 144 96.25) (end 133.75 96.25) (width 0.5) (layer "B.Cu") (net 1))
 (segment (start 144.5 80.785) (end 144.5 95.75) (width 0.5) (layer "B.Cu") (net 1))
 (segment (start 144.75 96) (end 144.5 95.75) (width 0.5) (layer "B.Cu") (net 1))
 (segment (start 159.725 90.244) (end 158.64737 90.244) (width 0.5) (layer "B.Cu") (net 1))
 (segment (start 132.54 70.46) (end 135.5 70.46) (width 0.5) (layer "B.Cu") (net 1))
 (segment (start 152.89137 96) (end 144.75 96) (width 0.5) (layer "B.Cu") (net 1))
 (segment (start 133.75 96.25) (end 132 94.5) (width 0.5) (layer "B.Cu") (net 1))
 (segment (start 144.5 95.75) (end 144 96.25) (width 0.5) (layer "B.Cu") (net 1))
 (segment (start 135 70.96) (end 135.5 70.46) (width 0.5) (layer "B.Cu") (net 1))
 (segment (start 132 71) (end 132.54 70.46) (width 0.5) (layer "B.Cu") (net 1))
 (segment (start 158.64737 90.244) (end 152.89137 96) (width 0.5) (layer "B.Cu") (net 1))
 (segment (start 135.5 70.46) (end 143.46 70.46) (width 0.5) (layer "B.Cu") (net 1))
 (segment (start 148.54 73) (end 151.15 75.61) (width 0.5) (layer "B.Cu") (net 9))
 (segment (start 151.29 75.75) (end 151.15 75.61) (width 0.5) (layer "B.Cu") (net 9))
 (segment (start 157.25 69.25) (end 157.25 75.75) (width 0.5) (layer "B.Cu") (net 9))
 (segment (start 157.25 75.75) (end 151.29 75.75) (width 0.5) (layer "B.Cu") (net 9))
 (segment (start 151.15 75.61) (end 151.15 80.785) (width 0.5) (layer "B.Cu") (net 9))
 (segment (start 148 65.5) (end 144 65.5) (width 0.5) (layer "F.Cu") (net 8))
 (segment (start 139 70.5) (end 139 83.5) (width 0.5) (layer "F.Cu") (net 8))
 (segment (start 139 83.5) (end 137.5 85) (width 0.5) (layer "F.Cu") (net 8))
 (segment (start 144 65.5) (end 139 70.5) (width 0.5) (layer "F.Cu") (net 8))
 (via (at 137.5 85) (size 2.5) (drill 0.3) (layers "F.Cu" "B.Cu") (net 8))
 (via (at 148 65.5) (size 2.5) (drill 0.3) (layers "F.Cu" "B.Cu") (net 8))
 (segment (start 146 67.5) (end 146 70.46) (width 0.5) (layer "B.Cu") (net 8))
 (segment (start 137.5 85) (end 137.905 84.595) (width 0.5) (layer "B.Cu") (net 8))
 (segment (start 148 65.5) (end 146 67.5) (width 0.5) (layer "B.Cu") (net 8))
 (segment (start 137.905 84.595) (end 141.85 84.595) (width 0.5) (layer "B.Cu") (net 8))
 (segment (start 139.1 81.1) (end 140.055 82.055) (width 0.5) (layer "B.Cu") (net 7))
 (segment (start 146 73) (end 146 73.222562) (width 0.5) (layer "B.Cu") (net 7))
 (segment (start 140.055 82.055) (end 141.85 82.055) (width 0.5) (layer "B.Cu") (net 7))
 (segment (start 146 73.222562) (end 139.1 80.122562) (width 0.5) (layer "B.Cu") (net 7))
 (segment (start 139.1 80.122562) (end 139.1 81.1) (width 0.5) (layer "B.Cu") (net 7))
 (segment (start 143.46 73) (end 138 78.46) (width 0.5) (layer "B.Cu") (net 6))
 (segment (start 138 82) (end 139.325 83.325) (width 0.5) (layer "B.Cu") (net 6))
 (segment (start 138 78.46) (end 138 82) (width 0.5) (layer "B.Cu") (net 6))
 (segment (start 139.325 83.325) (end 141.85 83.325) (width 0.5) (layer "B.Cu") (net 6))
 (segment (start 134.525 89) (end 134.525 92.425) (width 0.5) (layer "B.Cu") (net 10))
 (segment (start 134.525 92.425) (end 134.45 92.5) (width 0.5) (layer "B.Cu") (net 10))
 (segment (start 139.445 90.945) (end 137.5 89) (width 0.5) (layer "B.Cu") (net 11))
 (segment (start 141.85 90.945) (end 139.445 90.945) (width 0.5) (layer "B.Cu") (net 11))
 (segment (start 136.665151 87.135) (end 135 85.469849) (width 0.5) (layer "B.Cu") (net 13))
 (segment (start 141.85 87.135) (end 136.665151 87.135) (width 0.5) (layer "B.Cu") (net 13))
 (segment (start 135 85.469849) (end 135 80.9875) (width 0.5) (layer "B.Cu") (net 13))
 (segment (start 135 75.05) (end 135 78.0125) (width 0.5) (layer "B.Cu") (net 12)))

